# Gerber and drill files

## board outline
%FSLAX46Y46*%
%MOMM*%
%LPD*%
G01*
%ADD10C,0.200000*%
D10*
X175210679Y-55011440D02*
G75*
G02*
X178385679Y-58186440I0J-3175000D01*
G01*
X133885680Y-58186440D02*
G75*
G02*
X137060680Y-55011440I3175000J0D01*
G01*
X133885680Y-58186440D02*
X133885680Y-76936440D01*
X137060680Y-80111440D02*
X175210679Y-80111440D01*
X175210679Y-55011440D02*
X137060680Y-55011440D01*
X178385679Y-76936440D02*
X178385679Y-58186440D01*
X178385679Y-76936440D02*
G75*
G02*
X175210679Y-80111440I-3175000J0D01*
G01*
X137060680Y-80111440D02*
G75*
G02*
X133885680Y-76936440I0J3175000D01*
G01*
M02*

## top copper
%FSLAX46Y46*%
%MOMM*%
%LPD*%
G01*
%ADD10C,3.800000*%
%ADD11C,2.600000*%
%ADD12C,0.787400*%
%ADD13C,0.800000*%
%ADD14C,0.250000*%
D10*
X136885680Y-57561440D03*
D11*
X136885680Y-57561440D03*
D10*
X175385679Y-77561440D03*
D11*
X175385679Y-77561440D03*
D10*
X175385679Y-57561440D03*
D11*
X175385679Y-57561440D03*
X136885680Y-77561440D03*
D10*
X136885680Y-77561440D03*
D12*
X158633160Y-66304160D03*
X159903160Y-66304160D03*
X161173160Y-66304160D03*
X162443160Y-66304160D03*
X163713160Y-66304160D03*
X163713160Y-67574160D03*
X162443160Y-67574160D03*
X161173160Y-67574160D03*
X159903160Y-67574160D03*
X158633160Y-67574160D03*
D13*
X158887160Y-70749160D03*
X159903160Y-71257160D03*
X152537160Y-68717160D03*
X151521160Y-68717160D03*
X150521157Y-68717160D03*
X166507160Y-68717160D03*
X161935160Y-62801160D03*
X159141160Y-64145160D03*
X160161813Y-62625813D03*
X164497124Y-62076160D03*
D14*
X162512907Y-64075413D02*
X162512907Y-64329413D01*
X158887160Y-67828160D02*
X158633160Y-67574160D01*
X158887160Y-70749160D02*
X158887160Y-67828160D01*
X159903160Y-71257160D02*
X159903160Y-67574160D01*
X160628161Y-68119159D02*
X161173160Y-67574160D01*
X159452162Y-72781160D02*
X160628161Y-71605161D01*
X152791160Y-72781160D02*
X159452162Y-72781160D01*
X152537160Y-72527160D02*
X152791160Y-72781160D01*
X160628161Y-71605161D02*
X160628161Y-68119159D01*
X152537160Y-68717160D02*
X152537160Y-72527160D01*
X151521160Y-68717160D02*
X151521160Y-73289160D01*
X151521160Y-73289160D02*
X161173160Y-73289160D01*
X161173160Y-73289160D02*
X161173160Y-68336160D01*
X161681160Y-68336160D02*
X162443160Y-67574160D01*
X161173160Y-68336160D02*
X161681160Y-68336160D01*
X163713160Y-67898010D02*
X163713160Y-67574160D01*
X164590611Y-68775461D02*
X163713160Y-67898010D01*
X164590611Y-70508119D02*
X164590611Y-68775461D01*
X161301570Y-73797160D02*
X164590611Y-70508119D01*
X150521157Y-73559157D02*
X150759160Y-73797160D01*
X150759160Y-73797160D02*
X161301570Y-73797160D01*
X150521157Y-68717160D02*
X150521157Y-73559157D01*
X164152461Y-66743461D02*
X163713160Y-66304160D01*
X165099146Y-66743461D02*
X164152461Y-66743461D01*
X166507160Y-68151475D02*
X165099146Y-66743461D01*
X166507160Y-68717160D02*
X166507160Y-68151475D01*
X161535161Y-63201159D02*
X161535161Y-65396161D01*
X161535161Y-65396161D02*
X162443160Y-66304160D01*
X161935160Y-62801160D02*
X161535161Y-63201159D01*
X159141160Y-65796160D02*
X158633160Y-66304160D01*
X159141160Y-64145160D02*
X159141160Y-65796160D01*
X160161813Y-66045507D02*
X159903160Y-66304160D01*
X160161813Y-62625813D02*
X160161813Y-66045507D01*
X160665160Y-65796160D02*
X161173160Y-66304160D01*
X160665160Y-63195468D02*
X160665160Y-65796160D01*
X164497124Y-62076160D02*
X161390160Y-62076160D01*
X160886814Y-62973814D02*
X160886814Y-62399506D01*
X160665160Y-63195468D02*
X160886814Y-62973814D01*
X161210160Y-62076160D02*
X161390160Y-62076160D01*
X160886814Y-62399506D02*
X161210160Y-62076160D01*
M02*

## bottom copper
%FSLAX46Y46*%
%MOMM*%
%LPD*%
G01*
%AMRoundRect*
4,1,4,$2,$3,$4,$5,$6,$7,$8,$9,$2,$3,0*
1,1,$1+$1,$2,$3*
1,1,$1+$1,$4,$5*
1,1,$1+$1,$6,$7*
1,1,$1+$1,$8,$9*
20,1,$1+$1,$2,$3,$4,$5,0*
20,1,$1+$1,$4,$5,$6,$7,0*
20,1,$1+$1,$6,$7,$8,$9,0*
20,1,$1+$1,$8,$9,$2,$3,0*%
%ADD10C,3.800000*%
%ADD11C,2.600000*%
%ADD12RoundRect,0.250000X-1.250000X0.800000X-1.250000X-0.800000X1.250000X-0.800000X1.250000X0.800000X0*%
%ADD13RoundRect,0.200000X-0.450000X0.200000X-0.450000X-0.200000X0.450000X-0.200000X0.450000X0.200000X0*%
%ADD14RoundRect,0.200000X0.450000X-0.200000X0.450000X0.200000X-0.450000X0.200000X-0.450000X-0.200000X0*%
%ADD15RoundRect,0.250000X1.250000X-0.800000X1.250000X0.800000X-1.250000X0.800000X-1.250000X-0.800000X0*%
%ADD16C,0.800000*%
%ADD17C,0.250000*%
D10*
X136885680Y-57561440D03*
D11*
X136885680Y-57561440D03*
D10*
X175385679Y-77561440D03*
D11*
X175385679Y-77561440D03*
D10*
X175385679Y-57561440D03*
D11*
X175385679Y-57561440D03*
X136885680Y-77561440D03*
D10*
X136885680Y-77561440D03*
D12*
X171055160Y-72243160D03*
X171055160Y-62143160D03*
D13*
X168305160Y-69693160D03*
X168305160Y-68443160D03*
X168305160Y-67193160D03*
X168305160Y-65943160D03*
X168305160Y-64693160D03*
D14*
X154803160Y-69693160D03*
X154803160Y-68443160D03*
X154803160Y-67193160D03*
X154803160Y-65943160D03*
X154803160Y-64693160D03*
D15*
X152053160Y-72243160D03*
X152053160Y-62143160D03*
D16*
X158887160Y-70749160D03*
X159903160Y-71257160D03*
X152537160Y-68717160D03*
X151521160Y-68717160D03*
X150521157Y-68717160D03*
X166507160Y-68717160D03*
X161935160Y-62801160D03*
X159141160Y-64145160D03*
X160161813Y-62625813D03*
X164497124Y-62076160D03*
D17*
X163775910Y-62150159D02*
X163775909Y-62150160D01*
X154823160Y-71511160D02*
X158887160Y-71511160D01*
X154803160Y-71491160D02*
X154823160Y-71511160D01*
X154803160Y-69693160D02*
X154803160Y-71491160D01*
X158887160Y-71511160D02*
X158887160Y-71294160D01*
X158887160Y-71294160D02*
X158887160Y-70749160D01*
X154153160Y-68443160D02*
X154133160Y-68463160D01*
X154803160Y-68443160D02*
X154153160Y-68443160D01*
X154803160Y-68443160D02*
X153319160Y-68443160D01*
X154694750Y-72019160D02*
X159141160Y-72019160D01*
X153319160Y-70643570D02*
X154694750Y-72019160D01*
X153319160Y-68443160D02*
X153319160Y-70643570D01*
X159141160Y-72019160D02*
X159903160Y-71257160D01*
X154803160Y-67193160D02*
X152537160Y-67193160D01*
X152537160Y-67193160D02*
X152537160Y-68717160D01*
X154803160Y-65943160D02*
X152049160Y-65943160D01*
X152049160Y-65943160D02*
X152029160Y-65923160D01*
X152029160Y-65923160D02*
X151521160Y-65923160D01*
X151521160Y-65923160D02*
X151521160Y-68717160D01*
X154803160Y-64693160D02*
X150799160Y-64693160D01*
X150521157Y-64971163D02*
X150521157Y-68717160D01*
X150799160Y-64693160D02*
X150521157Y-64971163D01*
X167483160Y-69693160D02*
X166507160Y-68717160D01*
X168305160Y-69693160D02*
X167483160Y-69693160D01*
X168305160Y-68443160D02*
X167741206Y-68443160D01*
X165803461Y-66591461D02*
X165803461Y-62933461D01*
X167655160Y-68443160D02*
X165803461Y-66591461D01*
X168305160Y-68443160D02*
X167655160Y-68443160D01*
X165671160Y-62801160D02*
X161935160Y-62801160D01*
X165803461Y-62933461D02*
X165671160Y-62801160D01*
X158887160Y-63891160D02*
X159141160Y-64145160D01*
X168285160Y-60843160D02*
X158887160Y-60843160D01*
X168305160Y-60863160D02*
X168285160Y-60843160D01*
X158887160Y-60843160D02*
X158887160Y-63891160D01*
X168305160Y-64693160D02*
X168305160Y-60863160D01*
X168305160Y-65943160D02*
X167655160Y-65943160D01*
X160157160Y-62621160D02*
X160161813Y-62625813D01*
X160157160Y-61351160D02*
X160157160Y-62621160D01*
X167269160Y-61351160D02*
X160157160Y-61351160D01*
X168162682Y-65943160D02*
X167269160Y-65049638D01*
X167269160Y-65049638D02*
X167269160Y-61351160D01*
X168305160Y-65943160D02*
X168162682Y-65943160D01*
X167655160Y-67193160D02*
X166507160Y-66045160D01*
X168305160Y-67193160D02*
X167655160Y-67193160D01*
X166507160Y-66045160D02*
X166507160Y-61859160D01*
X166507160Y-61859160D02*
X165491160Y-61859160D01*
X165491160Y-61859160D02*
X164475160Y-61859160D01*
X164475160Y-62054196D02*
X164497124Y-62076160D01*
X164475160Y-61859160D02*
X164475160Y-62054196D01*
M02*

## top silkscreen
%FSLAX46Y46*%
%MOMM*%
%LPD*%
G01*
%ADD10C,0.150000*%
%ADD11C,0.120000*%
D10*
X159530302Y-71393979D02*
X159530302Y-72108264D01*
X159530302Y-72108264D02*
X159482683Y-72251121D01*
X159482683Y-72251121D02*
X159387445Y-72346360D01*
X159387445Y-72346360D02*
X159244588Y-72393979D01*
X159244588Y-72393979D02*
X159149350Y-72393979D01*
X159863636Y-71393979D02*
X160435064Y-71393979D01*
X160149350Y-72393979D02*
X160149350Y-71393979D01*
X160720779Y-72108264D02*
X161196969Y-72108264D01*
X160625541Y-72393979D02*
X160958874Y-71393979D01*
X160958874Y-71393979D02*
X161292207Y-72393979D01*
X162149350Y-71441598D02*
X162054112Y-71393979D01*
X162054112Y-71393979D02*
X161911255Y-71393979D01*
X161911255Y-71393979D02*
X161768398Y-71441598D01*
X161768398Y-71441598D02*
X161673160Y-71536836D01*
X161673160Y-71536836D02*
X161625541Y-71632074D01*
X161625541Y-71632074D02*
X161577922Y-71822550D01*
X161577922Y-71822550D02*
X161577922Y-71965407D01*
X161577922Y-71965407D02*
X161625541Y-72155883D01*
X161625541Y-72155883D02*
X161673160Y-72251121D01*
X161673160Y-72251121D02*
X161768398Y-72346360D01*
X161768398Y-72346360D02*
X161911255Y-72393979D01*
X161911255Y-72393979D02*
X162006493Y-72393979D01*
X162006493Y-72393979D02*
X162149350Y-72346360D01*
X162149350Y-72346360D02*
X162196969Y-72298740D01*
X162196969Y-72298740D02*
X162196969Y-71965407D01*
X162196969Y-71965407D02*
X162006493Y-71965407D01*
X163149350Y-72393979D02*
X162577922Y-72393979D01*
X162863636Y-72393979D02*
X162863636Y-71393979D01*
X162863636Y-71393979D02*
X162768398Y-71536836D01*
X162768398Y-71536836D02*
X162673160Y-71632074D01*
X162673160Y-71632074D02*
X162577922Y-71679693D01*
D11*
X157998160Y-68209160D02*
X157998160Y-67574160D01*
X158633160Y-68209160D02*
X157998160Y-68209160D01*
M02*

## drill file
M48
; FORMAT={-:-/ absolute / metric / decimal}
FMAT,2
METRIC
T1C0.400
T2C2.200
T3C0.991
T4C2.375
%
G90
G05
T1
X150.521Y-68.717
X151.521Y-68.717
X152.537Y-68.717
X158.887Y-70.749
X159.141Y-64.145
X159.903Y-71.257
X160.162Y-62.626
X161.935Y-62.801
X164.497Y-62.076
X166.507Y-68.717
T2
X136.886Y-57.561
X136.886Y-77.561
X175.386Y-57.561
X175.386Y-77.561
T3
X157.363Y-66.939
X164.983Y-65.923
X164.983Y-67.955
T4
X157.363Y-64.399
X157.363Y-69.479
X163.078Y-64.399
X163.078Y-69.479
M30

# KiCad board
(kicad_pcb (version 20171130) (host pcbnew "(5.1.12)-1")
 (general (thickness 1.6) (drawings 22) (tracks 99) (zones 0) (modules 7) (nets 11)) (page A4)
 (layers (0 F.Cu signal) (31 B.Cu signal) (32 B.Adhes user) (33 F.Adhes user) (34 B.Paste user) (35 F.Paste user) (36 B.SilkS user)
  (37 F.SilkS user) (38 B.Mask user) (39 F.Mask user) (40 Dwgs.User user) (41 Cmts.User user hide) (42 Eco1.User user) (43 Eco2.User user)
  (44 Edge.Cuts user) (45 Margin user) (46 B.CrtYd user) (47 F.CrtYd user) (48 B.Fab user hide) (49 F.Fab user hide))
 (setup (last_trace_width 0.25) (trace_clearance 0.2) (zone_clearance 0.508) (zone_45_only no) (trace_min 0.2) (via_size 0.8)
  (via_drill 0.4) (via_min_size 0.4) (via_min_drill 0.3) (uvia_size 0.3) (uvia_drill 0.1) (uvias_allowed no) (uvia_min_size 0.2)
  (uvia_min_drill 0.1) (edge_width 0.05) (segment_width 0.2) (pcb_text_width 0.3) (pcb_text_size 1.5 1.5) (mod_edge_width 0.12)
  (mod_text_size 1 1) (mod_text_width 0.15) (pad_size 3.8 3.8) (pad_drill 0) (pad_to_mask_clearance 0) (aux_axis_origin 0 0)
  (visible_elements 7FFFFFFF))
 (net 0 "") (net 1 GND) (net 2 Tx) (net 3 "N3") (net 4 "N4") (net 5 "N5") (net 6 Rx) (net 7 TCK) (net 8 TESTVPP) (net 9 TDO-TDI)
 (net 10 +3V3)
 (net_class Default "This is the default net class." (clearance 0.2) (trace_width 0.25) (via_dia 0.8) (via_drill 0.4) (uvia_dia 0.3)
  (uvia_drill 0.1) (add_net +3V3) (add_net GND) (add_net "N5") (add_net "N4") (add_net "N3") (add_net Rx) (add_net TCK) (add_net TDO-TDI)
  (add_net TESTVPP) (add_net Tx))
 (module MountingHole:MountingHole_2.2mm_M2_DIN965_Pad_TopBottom (layer F.Cu) (at 136.88568 57.56144)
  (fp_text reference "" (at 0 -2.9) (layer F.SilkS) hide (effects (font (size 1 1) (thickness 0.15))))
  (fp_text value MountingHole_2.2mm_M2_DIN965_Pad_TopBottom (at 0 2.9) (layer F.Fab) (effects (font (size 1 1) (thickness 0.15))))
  (pad 1 connect circle (at 0 0) (size 3.8 3.8) (layers B.Cu B.Mask))
  (pad 1 connect circle (at 0 0) (size 3.8 3.8) (layers F.Cu F.Mask))
  (pad 1 thru_hole circle (at 0 0) (size 2.6 2.6) (drill 2.2) (layers *.Cu *.Mask)))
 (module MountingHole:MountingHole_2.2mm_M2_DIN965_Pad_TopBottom (layer F.Cu) (at 175.385679 77.56144)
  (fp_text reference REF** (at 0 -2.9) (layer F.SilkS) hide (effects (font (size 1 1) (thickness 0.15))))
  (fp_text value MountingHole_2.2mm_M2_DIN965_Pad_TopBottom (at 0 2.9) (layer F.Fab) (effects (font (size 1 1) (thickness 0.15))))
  (pad 1 connect circle (at 0 0) (size 3.8 3.8) (layers B.Cu B.Mask))
  (pad 1 connect circle (at 0 0) (size 3.8 3.8) (layers F.Cu F.Mask))
  (pad 1 thru_hole circle (at 0 0) (size 2.6 2.6) (drill 2.2) (layers *.Cu *.Mask)))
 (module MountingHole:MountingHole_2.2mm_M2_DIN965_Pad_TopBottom (layer F.Cu) (at 175.385679 57.56144)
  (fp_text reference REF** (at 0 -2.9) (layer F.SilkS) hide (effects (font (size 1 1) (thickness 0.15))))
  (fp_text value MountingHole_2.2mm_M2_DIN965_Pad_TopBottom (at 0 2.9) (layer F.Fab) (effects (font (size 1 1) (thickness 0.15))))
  (pad 1 connect circle (at 0 0) (size 3.8 3.8) (layers B.Cu B.Mask))
  (pad 1 connect circle (at 0 0) (size 3.8 3.8) (layers F.Cu F.Mask))
  (pad 1 thru_hole circle (at 0 0) (size 2.6 2.6) (drill 2.2) (layers *.Cu *.Mask)))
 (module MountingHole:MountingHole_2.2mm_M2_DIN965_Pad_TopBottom (layer F.Cu) (at 136.88568 77.56144)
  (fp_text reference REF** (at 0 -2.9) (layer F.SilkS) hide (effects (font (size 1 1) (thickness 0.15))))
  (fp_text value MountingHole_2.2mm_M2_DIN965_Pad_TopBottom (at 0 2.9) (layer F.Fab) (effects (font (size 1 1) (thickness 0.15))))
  (pad 1 thru_hole circle (at 0 0) (size 2.6 2.6) (drill 2.2) (layers *.Cu *.Mask))
  (pad 1 connect circle (at 0 0) (size 3.8 3.8) (layers F.Cu F.Mask))
  (pad 1 connect circle (at 0 0) (size 3.8 3.8) (layers B.Cu B.Mask)))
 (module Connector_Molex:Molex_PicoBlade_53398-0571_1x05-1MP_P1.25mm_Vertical (layer B.Cu) (at 169.55516 67.19316 270)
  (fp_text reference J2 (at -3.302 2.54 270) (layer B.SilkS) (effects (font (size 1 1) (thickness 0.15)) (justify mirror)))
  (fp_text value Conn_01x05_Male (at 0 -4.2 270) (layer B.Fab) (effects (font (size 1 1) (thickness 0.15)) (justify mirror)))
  (pad MP smd roundrect (at 5.05 -1.5 270) (size 2.1 3) (layers B.Cu B.Paste B.Mask) (roundrect_rratio 0.119047619047619))
  (pad MP smd roundrect (at -5.05 -1.5 270) (size 2.1 3) (layers B.Cu B.Paste B.Mask) (roundrect_rratio 0.119047619047619))
  (pad 5 smd roundrect (at 2.5 1.25 270) (size 0.8 1.3) (layers B.Cu B.Paste B.Mask) (roundrect_rratio 0.25) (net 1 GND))
  (pad 4 smd roundrect (at 1.25 1.25 270) (size 0.8 1.3) (layers B.Cu B.Paste B.Mask) (roundrect_rratio 0.25) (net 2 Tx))
  (pad 3 smd roundrect (at 0 1.25 270) (size 0.8 1.3) (layers B.Cu B.Paste B.Mask) (roundrect_rratio 0.25) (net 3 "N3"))
  (pad 2 smd roundrect (at -1.25 1.25 270) (size 0.8 1.3) (layers B.Cu B.Paste B.Mask) (roundrect_rratio 0.25) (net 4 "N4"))
  (pad 1 smd roundrect (at -2.5 1.25 270) (size 0.8 1.3) (layers B.Cu B.Paste B.Mask) (roundrect_rratio 0.25) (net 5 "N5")))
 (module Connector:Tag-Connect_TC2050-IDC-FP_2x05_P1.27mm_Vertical (layer F.Cu) (at 161.17316 66.93916)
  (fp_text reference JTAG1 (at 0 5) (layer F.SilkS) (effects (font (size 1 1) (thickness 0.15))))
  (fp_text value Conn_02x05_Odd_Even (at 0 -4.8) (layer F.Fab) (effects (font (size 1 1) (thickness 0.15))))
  (fp_line (start -3.175 1.27) (end -3.175 0.635) (layer F.SilkS) (width 0.12))
  (fp_line (start -2.54 1.27) (end -3.175 1.27) (layer F.SilkS) (width 0.12))
  (pad "" np_thru_hole circle (at 1.905 -2.54) (size 2.3749 2.3749) (drill 2.3749) (layers *.Cu *.Mask))
  (pad "" np_thru_hole circle (at 1.905 2.54) (size 2.3749 2.3749) (drill 2.3749) (layers *.Cu *.Mask))
  (pad "" np_thru_hole circle (at -3.81 2.54) (size 2.3749 2.3749) (drill 2.3749) (layers *.Cu *.Mask))
  (pad "" np_thru_hole circle (at -3.81 -2.54) (size 2.3749 2.3749) (drill 2.3749) (layers *.Cu *.Mask))
  (pad 10 connect circle (at -2.54 -0.635) (size 0.7874 0.7874) (layers F.Cu F.Mask) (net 5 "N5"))
  (pad 9 connect circle (at -1.27 -0.635) (size 0.7874 0.7874) (layers F.Cu F.Mask) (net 4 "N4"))
  (pad 8 connect circle (at 0 -0.635) (size 0.7874 0.7874) (layers F.Cu F.Mask) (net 3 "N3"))
  (pad 7 connect circle (at 1.27 -0.635) (size 0.7874 0.7874) (layers F.Cu F.Mask) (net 2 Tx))
  (pad 6 connect circle (at 2.54 -0.635) (size 0.7874 0.7874) (layers F.Cu F.Mask) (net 1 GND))
  (pad 5 connect circle (at 2.54 0.635) (size 0.7874 0.7874) (layers F.Cu F.Mask) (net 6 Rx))
  (pad 4 connect circle (at 1.27 0.635) (size 0.7874 0.7874) (layers F.Cu F.Mask) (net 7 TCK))
  (pad 3 connect circle (at 0 0.635) (size 0.7874 0.7874) (layers F.Cu F.Mask) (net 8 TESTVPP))
  (pad 2 connect circle (at -1.27 0.635) (size 0.7874 0.7874) (layers F.Cu F.Mask) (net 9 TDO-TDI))
  (pad 1 connect circle (at -2.54 0.635) (size 0.7874 0.7874) (layers F.Cu F.Mask) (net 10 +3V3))
  (pad "" np_thru_hole circle (at -3.81 0) (size 0.9906 0.9906) (drill 0.9906) (layers *.Cu *.Mask))
  (pad "" np_thru_hole circle (at 3.81 1.016) (size 0.9906 0.9906) (drill 0.9906) (layers *.Cu *.Mask))
  (pad "" np_thru_hole circle (at 3.81 -1.016) (size 0.9906 0.9906) (drill 0.9906) (layers *.Cu *.Mask)))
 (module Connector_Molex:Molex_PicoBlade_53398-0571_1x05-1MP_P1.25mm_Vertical (layer B.Cu) (at 153.55316 67.19316 90)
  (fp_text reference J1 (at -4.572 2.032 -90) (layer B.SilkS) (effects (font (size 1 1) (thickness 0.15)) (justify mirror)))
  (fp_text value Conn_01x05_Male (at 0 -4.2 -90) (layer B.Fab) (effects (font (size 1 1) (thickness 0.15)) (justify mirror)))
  (pad 1 smd roundrect (at -2.5 1.25 90) (size 0.8 1.3) (layers B.Cu B.Paste B.Mask) (roundrect_rratio 0.25) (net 10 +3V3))
  (pad 2 smd roundrect (at -1.25 1.25 90) (size 0.8 1.3) (layers B.Cu B.Paste B.Mask) (roundrect_rratio 0.25) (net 9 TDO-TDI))
  (pad 3 smd roundrect (at 0 1.25 90) (size 0.8 1.3) (layers B.Cu B.Paste B.Mask) (roundrect_rratio 0.25) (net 8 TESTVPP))
  (pad 4 smd roundrect (at 1.25 1.25 90) (size 0.8 1.3) (layers B.Cu B.Paste B.Mask) (roundrect_rratio 0.25) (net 7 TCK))
  (pad 5 smd roundrect (at 2.5 1.25 90) (size 0.8 1.3) (layers B.Cu B.Paste B.Mask) (roundrect_rratio 0.25) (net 6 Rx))
  (pad MP smd roundrect (at -5.05 -1.5 90) (size 2.1 3) (layers B.Cu B.Paste B.Mask) (roundrect_rratio 0.119047619047619))
  (pad MP smd roundrect (at 5.05 -1.5 90) (size 2.1 3) (layers B.Cu B.Paste B.Mask) (roundrect_rratio 0.119047619047619)))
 (gr_arc (start 175.210679 58.18644) (end 178.385679 58.18644) (angle -90) (layer Edge.Cuts) (width 0.2))
 (gr_arc (start 137.06068 58.18644) (end 137.06068 55.01144) (angle -90) (layer Edge.Cuts) (width 0.2))
 (gr_line (start 133.88568 58.18644) (end 133.88568 76.93644) (layer Edge.Cuts) (width 0.2))
 (gr_line (start 137.06068 80.11144) (end 175.210679 80.11144) (layer Edge.Cuts) (width 0.2))
 (gr_line (start 175.210679 55.01144) (end 137.06068 55.01144) (layer Edge.Cuts) (width 0.2))
 (gr_line (start 178.385679 76.93644) (end 178.385679 58.18644) (layer Edge.Cuts) (width 0.2))
 (gr_arc (start 175.210679 76.93644) (end 175.210679 80.11144) (angle -90) (layer Edge.Cuts) (width 0.2))
 (gr_arc (start 137.06068 76.93644) (end 133.88568 76.93644) (angle -90) (layer Edge.Cuts) (width 0.2))
 (segment (start 162.512907 64.075413) (end 162.512907 64.329413) (width 0.25) (layer F.Cu) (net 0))
 (segment (start 163.77591 62.150159) (end 163.775909 62.15016) (width 0.25) (layer B.Cu) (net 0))
 (segment (start 154.82316 71.51116) (end 158.88716 71.51116) (width 0.25) (layer B.Cu) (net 10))
 (segment (start 154.80316 71.49116) (end 154.82316 71.51116) (width 0.25) (layer B.Cu) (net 10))
 (segment (start 154.80316 69.69316) (end 154.80316 71.49116) (width 0.25) (layer B.Cu) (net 10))
 (segment (start 158.88716 71.51116) (end 158.88716 71.29416) (width 0.25) (layer B.Cu) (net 10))
 (via (at 158.88716 70.74916) (size 0.8) (drill 0.4) (layers F.Cu B.Cu) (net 10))
 (segment (start 158.88716 71.29416) (end 158.88716 70.74916) (width 0.25) (layer B.Cu) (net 10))
 (segment (start 158.88716 67.82816) (end 158.63316 67.57416) (width 0.25) (layer F.Cu) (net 10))
 (segment (start 158.88716 70.74916) (end 158.88716 67.82816) (width 0.25) (layer F.Cu) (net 10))
 (segment (start 154.15316 68.44316) (end 154.13316 68.46316) (width 0.25) (layer B.Cu) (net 9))
 (segment (start 154.80316 68.44316) (end 154.15316 68.44316) (width 0.25) (layer B.Cu) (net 9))
 (segment (start 154.80316 68.44316) (end 153.31916 68.44316) (width 0.25) (layer B.Cu) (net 9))
 (segment (start 154.69475 72.01916) (end 159.14116 72.01916) (width 0.25) (layer B.Cu) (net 9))
 (segment (start 153.31916 70.64357) (end 154.69475 72.01916) (width 0.25) (layer B.Cu) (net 9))
 (segment (start 153.31916 68.44316) (end 153.31916 70.64357) (width 0.25) (layer B.Cu) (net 9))
 (via (at 159.90316 71.25716) (size 0.8) (drill 0.4) (layers F.Cu B.Cu) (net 9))
 (segment (start 159.14116 72.01916) (end 159.90316 71.25716) (width 0.25) (layer B.Cu) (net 9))
 (segment (start 159.90316 71.25716) (end 159.90316 67.57416) (width 0.25) (layer F.Cu) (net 9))
 (segment (start 154.80316 67.19316) (end 152.53716 67.19316) (width 0.25) (layer B.Cu) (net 8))
 (via (at 152.53716 68.71716) (size 0.8) (drill 0.4) (layers F.Cu B.Cu) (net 8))
 (segment (start 152.53716 67.19316) (end 152.53716 68.71716) (width 0.25) (layer B.Cu) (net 8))
 (segment (start 160.628161 68.119159) (end 161.17316 67.57416) (width 0.25) (layer F.Cu) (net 8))
 (segment (start 159.452162 72.78116) (end 160.628161 71.605161) (width 0.25) (layer F.Cu) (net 8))
 (segment (start 152.79116 72.78116) (end 159.452162 72.78116) (width 0.25) (layer F.Cu) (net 8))
 (segment (start 152.53716 72.52716) (end 152.79116 72.78116) (width 0.25) (layer F.Cu) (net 8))
 (segment (start 160.628161 71.605161) (end 160.628161 68.119159) (width 0.25) (layer F.Cu) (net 8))
 (segment (start 152.53716 68.71716) (end 152.53716 72.52716) (width 0.25) (layer F.Cu) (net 8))
 (segment (start 154.80316 65.94316) (end 152.04916 65.94316) (width 0.25) (layer B.Cu) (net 7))
 (segment (start 152.04916 65.94316) (end 152.02916 65.92316) (width 0.25) (layer B.Cu) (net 7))
 (segment (start 152.02916 65.92316) (end 151.52116 65.92316) (width 0.25) (layer B.Cu) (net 7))
 (via (at 151.52116 68.71716) (size 0.8) (drill 0.4) (layers F.Cu B.Cu) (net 7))
 (segment (start 151.52116 65.92316) (end 151.52116 68.71716) (width 0.25) (layer B.Cu) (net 7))
 (segment (start 151.52116 68.71716) (end 151.52116 73.28916) (width 0.25) (layer F.Cu) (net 7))
 (segment (start 151.52116 73.28916) (end 161.17316 73.28916) (width 0.25) (layer F.Cu) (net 7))
 (segment (start 161.17316 73.28916) (end 161.17316 68.33616) (width 0.25) (layer F.Cu) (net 7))
 (segment (start 161.68116 68.33616) (end 162.44316 67.57416) (width 0.25) (layer F.Cu) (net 7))
 (segment (start 161.17316 68.33616) (end 161.68116 68.33616) (width 0.25) (layer F.Cu) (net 7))
 (segment (start 154.80316 64.69316) (end 150.79916 64.69316) (width 0.25) (layer B.Cu) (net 6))
 (via (at 150.521157 68.71716) (size 0.8) (drill 0.4) (layers F.Cu B.Cu) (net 6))
 (segment (start 150.521157 64.971163) (end 150.521157 68.71716) (width 0.25) (layer B.Cu) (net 6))
 (segment (start 150.79916 64.69316) (end 150.521157 64.971163) (width 0.25) (layer B.Cu) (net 6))
 (segment (start 163.71316 67.89801) (end 163.71316 67.57416) (width 0.25) (layer F.Cu) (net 6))
 (segment (start 164.590611 68.775461) (end 163.71316 67.89801) (width 0.25) (layer F.Cu) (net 6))
 (segment (start 164.590611 70.508119) (end 164.590611 68.775461) (width 0.25) (layer F.Cu) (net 6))
 (segment (start 161.30157 73.79716) (end 164.590611 70.508119) (width 0.25) (layer F.Cu) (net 6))
 (segment (start 150.521157 73.559157) (end 150.75916 73.79716) (width 0.25) (layer F.Cu) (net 6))
 (segment (start 150.75916 73.79716) (end 161.30157 73.79716) (width 0.25) (layer F.Cu) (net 6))
 (segment (start 150.521157 68.71716) (end 150.521157 73.559157) (width 0.25) (layer F.Cu) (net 6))
 (via (at 166.50716 68.71716) (size 0.8) (drill 0.4) (layers F.Cu B.Cu) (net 1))
 (segment (start 167.48316 69.69316) (end 166.50716 68.71716) (width 0.25) (layer B.Cu) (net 1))
 (segment (start 168.30516 69.69316) (end 167.48316 69.69316) (width 0.25) (layer B.Cu) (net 1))
 (segment (start 164.152461 66.743461) (end 163.71316 66.30416) (width 0.25) (layer F.Cu) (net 1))
 (segment (start 165.099146 66.743461) (end 164.152461 66.743461) (width 0.25) (layer F.Cu) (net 1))
 (segment (start 166.50716 68.151475) (end 165.099146 66.743461) (width 0.25) (layer F.Cu) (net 1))
 (segment (start 166.50716 68.71716) (end 166.50716 68.151475) (width 0.25) (layer F.Cu) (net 1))
 (segment (start 168.30516 68.44316) (end 167.741206 68.44316) (width 0.25) (layer B.Cu) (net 2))
 (segment (start 165.803461 66.591461) (end 165.803461 62.933461) (width 0.25) (layer B.Cu) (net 2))
 (segment (start 167.65516 68.44316) (end 165.803461 66.591461) (width 0.25) (layer B.Cu) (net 2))
 (segment (start 168.30516 68.44316) (end 167.65516 68.44316) (width 0.25) (layer B.Cu) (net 2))
 (segment (start 165.67116 62.80116) (end 161.93516 62.80116) (width 0.25) (layer B.Cu) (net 2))
 (via (at 161.93516 62.80116) (size 0.8) (drill 0.4) (layers F.Cu B.Cu) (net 2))
 (segment (start 165.803461 62.933461) (end 165.67116 62.80116) (width 0.25) (layer B.Cu) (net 2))
 (segment (start 161.535161 63.201159) (end 161.535161 65.396161) (width 0.25) (layer F.Cu) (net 2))
 (segment (start 161.535161 65.396161) (end 162.44316 66.30416) (width 0.25) (layer F.Cu) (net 2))
 (segment (start 161.93516 62.80116) (end 161.535161 63.201159) (width 0.25) (layer F.Cu) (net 2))
 (via (at 159.14116 64.14516) (size 0.8) (drill 0.4) (layers F.Cu B.Cu) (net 5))
 (segment (start 159.14116 65.79616) (end 158.63316 66.30416) (width 0.25) (layer F.Cu) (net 5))
 (segment (start 159.14116 64.14516) (end 159.14116 65.79616) (width 0.25) (layer F.Cu) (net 5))
 (segment (start 158.88716 63.89116) (end 159.14116 64.14516) (width 0.25) (layer B.Cu) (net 5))
 (segment (start 168.28516 60.84316) (end 158.88716 60.84316) (width 0.25) (layer B.Cu) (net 5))
 (segment (start 168.30516 60.86316) (end 168.28516 60.84316) (width 0.25) (layer B.Cu) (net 5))
 (segment (start 158.88716 60.84316) (end 158.88716 63.89116) (width 0.25) (layer B.Cu) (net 5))
 (segment (start 168.30516 64.69316) (end 168.30516 60.86316) (width 0.25) (layer B.Cu) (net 5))
 (segment (start 168.30516 65.94316) (end 167.65516 65.94316) (width 0.25) (layer B.Cu) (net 4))
 (via (at 160.161813 62.625813) (size 0.8) (drill 0.4) (layers F.Cu B.Cu) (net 4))
 (segment (start 160.161813 66.045507) (end 159.90316 66.30416) (width 0.25) (layer F.Cu) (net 4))
 (segment (start 160.161813 62.625813) (end 160.161813 66.045507) (width 0.25) (layer F.Cu) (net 4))
 (segment (start 160.15716 62.62116) (end 160.161813 62.625813) (width 0.25) (layer B.Cu) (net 4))
 (segment (start 160.15716 61.35116) (end 160.15716 62.62116) (width 0.25) (layer B.Cu) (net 4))
 (segment (start 167.26916 61.35116) (end 160.15716 61.35116) (width 0.25) (layer B.Cu) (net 4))
 (segment (start 168.162682 65.94316) (end 167.26916 65.049638) (width 0.25) (layer B.Cu) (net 4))
 (segment (start 167.26916 65.049638) (end 167.26916 61.35116) (width 0.25) (layer B.Cu) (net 4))
 (segment (start 168.30516 65.94316) (end 168.162682 65.94316) (width 0.25) (layer B.Cu) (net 4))
 (segment (start 167.65516 67.19316) (end 166.50716 66.04516) (width 0.25) (layer B.Cu) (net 3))
 (segment (start 168.30516 67.19316) (end 167.65516 67.19316) (width 0.25) (layer B.Cu) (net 3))
 (segment (start 166.50716 66.04516) (end 166.50716 61.85916) (width 0.25) (layer B.Cu) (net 3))
 (segment (start 166.50716 61.85916) (end 165.49116 61.85916) (width 0.25) (layer B.Cu) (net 3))
 (segment (start 165.49116 61.85916) (end 164.47516 61.85916) (width 0.25) (layer B.Cu) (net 3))
 (via (at 164.497124 62.07616) (size 0.8) (drill 0.4) (layers F.Cu B.Cu) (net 3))
 (segment (start 164.47516 62.054196) (end 164.497124 62.07616) (width 0.25) (layer B.Cu) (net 3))
 (segment (start 164.47516 61.85916) (end 164.47516 62.054196) (width 0.25) (layer B.Cu) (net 3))
 (segment (start 160.66516 65.79616) (end 161.17316 66.30416) (width 0.25) (layer F.Cu) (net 3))
 (segment (start 160.66516 63.195468) (end 160.66516 65.79616) (width 0.25) (layer F.Cu) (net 3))
 (segment (start 164.497124 62.07616) (end 161.39016 62.07616) (width 0.25) (layer F.Cu) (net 3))
 (segment (start 160.886814 62.973814) (end 160.886814 62.399506) (width 0.25) (layer F.Cu) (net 3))
 (segment (start 160.66516 63.195468) (end 160.886814 62.973814) (width 0.25) (layer F.Cu) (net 3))
 (segment (start 161.21016 62.07616) (end 161.39016 62.07616) (width 0.25) (layer F.Cu) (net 3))
 (segment (start 160.886814 62.399506) (end 161.21016 62.07616) (width 0.25) (layer F.Cu) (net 3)))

